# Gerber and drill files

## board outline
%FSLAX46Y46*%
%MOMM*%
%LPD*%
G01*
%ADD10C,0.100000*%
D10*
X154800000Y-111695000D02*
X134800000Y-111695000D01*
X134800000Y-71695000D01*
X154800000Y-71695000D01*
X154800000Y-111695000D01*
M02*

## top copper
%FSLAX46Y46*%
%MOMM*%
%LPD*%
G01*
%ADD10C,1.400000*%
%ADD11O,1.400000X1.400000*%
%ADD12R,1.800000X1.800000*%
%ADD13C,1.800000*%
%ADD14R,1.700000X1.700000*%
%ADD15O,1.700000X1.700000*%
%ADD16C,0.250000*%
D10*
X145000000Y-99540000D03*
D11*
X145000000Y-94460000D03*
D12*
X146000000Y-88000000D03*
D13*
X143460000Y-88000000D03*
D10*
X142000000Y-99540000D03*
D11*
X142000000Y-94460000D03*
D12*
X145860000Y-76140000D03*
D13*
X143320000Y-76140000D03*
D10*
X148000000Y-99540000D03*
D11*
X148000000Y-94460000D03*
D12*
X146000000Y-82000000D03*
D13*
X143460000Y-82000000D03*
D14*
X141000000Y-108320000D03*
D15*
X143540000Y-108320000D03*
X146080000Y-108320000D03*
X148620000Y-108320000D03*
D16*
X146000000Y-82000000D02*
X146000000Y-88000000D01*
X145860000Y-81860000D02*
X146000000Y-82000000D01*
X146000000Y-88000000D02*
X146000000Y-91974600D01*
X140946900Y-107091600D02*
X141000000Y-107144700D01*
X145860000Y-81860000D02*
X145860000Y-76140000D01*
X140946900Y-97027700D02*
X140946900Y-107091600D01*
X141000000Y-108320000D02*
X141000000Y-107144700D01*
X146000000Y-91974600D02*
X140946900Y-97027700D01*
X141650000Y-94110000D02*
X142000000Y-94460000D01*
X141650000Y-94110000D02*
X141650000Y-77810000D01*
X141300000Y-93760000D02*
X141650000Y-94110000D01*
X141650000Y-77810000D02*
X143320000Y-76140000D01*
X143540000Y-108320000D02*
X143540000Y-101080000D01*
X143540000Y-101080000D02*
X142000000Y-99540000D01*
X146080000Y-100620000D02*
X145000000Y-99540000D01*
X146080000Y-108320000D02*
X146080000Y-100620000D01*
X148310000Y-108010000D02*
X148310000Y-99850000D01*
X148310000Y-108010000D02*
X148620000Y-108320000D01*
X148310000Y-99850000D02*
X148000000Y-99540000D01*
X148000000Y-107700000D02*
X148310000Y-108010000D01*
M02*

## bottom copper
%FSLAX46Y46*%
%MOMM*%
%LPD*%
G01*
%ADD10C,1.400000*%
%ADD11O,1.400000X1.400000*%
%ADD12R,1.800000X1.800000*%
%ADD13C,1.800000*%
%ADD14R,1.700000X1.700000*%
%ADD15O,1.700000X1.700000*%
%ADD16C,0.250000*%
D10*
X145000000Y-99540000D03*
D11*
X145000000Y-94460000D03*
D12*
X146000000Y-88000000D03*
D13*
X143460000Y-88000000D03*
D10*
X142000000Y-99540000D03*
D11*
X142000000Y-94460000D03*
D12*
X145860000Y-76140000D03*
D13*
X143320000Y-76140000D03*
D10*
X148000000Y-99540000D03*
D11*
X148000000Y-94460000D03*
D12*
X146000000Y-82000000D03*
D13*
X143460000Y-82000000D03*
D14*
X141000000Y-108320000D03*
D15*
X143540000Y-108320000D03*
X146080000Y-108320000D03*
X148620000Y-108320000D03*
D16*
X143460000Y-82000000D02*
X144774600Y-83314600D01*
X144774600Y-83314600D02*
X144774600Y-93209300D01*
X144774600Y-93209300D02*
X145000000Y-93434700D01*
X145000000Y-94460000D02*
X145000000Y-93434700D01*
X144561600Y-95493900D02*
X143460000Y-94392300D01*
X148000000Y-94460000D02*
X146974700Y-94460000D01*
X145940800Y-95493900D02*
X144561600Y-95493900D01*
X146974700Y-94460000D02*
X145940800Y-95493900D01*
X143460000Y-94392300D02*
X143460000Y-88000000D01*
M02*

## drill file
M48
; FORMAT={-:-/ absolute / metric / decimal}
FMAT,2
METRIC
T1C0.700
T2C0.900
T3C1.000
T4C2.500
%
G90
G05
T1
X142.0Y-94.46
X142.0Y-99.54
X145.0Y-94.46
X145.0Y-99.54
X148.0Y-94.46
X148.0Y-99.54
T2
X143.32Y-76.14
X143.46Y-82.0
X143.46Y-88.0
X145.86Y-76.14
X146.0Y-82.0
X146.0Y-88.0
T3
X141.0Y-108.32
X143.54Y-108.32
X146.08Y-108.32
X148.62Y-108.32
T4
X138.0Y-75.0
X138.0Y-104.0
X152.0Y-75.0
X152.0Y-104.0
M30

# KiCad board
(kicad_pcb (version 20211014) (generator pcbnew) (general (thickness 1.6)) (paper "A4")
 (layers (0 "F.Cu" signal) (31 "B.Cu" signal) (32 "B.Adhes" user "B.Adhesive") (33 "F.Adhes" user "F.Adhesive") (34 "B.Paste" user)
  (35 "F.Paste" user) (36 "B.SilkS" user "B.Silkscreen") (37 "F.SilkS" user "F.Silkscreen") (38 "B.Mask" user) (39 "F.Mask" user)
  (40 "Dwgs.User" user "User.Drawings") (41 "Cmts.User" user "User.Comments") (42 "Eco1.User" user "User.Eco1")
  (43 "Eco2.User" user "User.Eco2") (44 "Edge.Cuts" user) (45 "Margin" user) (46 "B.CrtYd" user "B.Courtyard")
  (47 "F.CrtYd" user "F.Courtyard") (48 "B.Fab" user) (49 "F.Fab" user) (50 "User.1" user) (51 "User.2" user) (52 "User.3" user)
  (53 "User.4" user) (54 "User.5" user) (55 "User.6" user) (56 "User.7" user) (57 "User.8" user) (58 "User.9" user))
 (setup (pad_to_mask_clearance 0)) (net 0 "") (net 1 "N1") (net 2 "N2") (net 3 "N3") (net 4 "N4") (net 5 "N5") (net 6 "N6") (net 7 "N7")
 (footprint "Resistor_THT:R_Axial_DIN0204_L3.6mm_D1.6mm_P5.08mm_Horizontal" (layer "F.Cu") (at 145 99.54 90)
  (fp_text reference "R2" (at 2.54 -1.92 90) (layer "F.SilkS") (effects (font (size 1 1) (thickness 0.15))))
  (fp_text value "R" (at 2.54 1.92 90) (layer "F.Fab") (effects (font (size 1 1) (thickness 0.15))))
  (pad "1" thru_hole circle (at 0 0 90) (size 1.4 1.4) (drill 0.7) (layers *.Cu *.Mask) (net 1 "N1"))
  (pad "2" thru_hole oval (at 5.08 0 90) (size 1.4 1.4) (drill 0.7) (layers *.Cu *.Mask) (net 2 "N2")))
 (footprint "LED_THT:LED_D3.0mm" (layer "F.Cu") (at 146 88 180)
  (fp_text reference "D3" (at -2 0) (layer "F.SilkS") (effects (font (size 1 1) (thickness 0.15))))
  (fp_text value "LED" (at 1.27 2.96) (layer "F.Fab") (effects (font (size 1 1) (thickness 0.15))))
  (pad "1" thru_hole rect (at 0 0 180) (size 1.8 1.8) (drill 0.9) (layers *.Cu *.Mask) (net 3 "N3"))
  (pad "2" thru_hole circle (at 2.54 0 180) (size 1.8 1.8) (drill 0.9) (layers *.Cu *.Mask) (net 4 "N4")))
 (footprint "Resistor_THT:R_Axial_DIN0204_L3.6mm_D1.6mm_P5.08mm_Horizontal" (layer "F.Cu") (at 142 99.54 90)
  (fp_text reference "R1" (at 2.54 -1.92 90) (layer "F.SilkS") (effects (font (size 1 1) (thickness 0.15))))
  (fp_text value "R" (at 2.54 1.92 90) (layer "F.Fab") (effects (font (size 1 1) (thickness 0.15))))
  (pad "1" thru_hole circle (at 0 0 90) (size 1.4 1.4) (drill 0.7) (layers *.Cu *.Mask) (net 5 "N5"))
  (pad "2" thru_hole oval (at 5.08 0 90) (size 1.4 1.4) (drill 0.7) (layers *.Cu *.Mask) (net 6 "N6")))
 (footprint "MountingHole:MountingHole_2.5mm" (layer "F.Cu") (at 152 75)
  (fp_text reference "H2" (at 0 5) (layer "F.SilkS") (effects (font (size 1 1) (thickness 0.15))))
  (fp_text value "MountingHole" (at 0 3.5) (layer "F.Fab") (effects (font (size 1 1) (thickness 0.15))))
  (pad "" np_thru_hole circle (at 0 0) (size 2.5 2.5) (drill 2.5) (layers *.Cu *.Mask)))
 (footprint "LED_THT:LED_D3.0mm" (layer "F.Cu") (at 145.86 76.14 180)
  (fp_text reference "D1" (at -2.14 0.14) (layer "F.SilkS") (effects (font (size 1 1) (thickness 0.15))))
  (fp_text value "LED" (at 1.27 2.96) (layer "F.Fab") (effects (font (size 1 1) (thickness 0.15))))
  (pad "1" thru_hole rect (at 0 0 180) (size 1.8 1.8) (drill 0.9) (layers *.Cu *.Mask) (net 3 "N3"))
  (pad "2" thru_hole circle (at 2.54 0 180) (size 1.8 1.8) (drill 0.9) (layers *.Cu *.Mask) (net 6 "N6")))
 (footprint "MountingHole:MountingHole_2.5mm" (layer "F.Cu") (at 138 104)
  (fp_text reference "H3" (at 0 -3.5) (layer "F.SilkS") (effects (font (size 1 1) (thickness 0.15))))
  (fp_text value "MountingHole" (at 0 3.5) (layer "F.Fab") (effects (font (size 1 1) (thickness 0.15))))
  (pad "" np_thru_hole circle (at 0 0) (size 2.5 2.5) (drill 2.5) (layers *.Cu *.Mask)))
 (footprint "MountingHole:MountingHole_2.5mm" (layer "F.Cu") (at 152 104)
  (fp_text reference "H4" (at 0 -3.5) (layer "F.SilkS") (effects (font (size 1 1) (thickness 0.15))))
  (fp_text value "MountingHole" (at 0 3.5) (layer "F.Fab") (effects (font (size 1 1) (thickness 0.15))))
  (pad "" np_thru_hole circle (at 0 0) (size 2.5 2.5) (drill 2.5) (layers *.Cu *.Mask)))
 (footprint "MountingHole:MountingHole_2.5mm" (layer "F.Cu") (at 138 75)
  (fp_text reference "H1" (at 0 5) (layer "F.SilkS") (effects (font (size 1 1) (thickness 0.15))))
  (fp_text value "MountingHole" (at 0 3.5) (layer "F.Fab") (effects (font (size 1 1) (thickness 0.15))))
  (pad "" np_thru_hole circle (at 0 0) (size 2.5 2.5) (drill 2.5) (layers *.Cu *.Mask)))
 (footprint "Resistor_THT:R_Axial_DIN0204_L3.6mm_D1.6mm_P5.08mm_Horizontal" (layer "F.Cu") (at 148 99.54 90)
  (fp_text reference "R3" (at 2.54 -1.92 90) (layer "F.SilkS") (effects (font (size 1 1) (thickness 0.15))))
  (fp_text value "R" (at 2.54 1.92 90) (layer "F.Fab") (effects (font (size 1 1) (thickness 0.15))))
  (pad "1" thru_hole circle (at 0 0 90) (size 1.4 1.4) (drill 0.7) (layers *.Cu *.Mask) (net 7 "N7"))
  (pad "2" thru_hole oval (at 5.08 0 90) (size 1.4 1.4) (drill 0.7) (layers *.Cu *.Mask) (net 4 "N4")))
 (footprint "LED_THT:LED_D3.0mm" (layer "F.Cu") (at 146 82 180)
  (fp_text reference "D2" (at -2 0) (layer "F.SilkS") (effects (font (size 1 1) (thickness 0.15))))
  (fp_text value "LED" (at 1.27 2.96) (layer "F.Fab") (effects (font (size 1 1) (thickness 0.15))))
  (pad "1" thru_hole rect (at 0 0 180) (size 1.8 1.8) (drill 0.9) (layers *.Cu *.Mask) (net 3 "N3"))
  (pad "2" thru_hole circle (at 2.54 0 180) (size 1.8 1.8) (drill 0.9) (layers *.Cu *.Mask) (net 2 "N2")))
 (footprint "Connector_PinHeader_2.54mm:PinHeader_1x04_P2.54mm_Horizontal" (layer "B.Cu") (at 141 108.32 -90)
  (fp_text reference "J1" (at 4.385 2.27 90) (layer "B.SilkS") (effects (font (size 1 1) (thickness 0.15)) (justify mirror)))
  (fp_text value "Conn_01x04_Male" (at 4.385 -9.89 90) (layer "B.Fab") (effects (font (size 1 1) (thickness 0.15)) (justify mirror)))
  (pad "1" thru_hole rect (at 0 0 270) (size 1.7 1.7) (drill 1) (layers *.Cu *.Mask) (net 3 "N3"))
  (pad "2" thru_hole oval (at 0 -2.54 270) (size 1.7 1.7) (drill 1) (layers *.Cu *.Mask) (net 5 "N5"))
  (pad "3" thru_hole oval (at 0 -5.08 270) (size 1.7 1.7) (drill 1) (layers *.Cu *.Mask) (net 1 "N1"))
  (pad "4" thru_hole oval (at 0 -7.62 270) (size 1.7 1.7) (drill 1) (layers *.Cu *.Mask) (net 7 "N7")))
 (gr_poly (pts (xy 154.8 111.695) (xy 134.8 111.695) (xy 134.8 71.695) (xy 154.8 71.695)) (layer "Edge.Cuts") (width 0.1) (fill none))
 (segment (start 146 82) (end 146 88) (width 0.25) (layer "F.Cu") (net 3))
 (segment (start 145.86 81.86) (end 146 82) (width 0.25) (layer "F.Cu") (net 3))
 (segment (start 146 88) (end 146 91.9746) (width 0.25) (layer "F.Cu") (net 3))
 (segment (start 140.9469 107.0916) (end 141 107.1447) (width 0.25) (layer "F.Cu") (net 3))
 (segment (start 145.86 81.86) (end 145.86 76.14) (width 0.25) (layer "F.Cu") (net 3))
 (segment (start 140.9469 97.0277) (end 140.9469 107.0916) (width 0.25) (layer "F.Cu") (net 3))
 (segment (start 141 108.32) (end 141 107.1447) (width 0.25) (layer "F.Cu") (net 3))
 (segment (start 146 91.9746) (end 140.9469 97.0277) (width 0.25) (layer "F.Cu") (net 3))
 (segment (start 141.65 94.11) (end 142 94.46) (width 0.25) (layer "F.Cu") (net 6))
 (segment (start 141.65 94.11) (end 141.65 77.81) (width 0.25) (layer "F.Cu") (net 6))
 (segment (start 141.3 93.76) (end 141.65 94.11) (width 0.25) (layer "F.Cu") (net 6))
 (segment (start 141.65 77.81) (end 143.32 76.14) (width 0.25) (layer "F.Cu") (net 6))
 (segment (start 143.46 82) (end 144.7746 83.3146) (width 0.25) (layer "B.Cu") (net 2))
 (segment (start 144.7746 83.3146) (end 144.7746 93.2093) (width 0.25) (layer "B.Cu") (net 2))
 (segment (start 144.7746 93.2093) (end 145 93.4347) (width 0.25) (layer "B.Cu") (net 2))
 (segment (start 145 94.46) (end 145 93.4347) (width 0.25) (layer "B.Cu") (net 2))
 (segment (start 144.5616 95.4939) (end 143.46 94.3923) (width 0.25) (layer "B.Cu") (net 4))
 (segment (start 148 94.46) (end 146.9747 94.46) (width 0.25) (layer "B.Cu") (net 4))
 (segment (start 145.9408 95.4939) (end 144.5616 95.4939) (width 0.25) (layer "B.Cu") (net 4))
 (segment (start 146.9747 94.46) (end 145.9408 95.4939) (width 0.25) (layer "B.Cu") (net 4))
 (segment (start 143.46 94.3923) (end 143.46 88) (width 0.25) (layer "B.Cu") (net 4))
 (segment (start 143.54 108.32) (end 143.54 101.08) (width 0.25) (layer "F.Cu") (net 5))
 (segment (start 143.54 101.08) (end 142 99.54) (width 0.25) (layer "F.Cu") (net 5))
 (segment (start 146.08 100.62) (end 145 99.54) (width 0.25) (layer "F.Cu") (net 1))
 (segment (start 146.08 108.32) (end 146.08 100.62) (width 0.25) (layer "F.Cu") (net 1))
 (segment (start 148.31 108.01) (end 148.31 99.85) (width 0.25) (layer "F.Cu") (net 7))
 (segment (start 148.31 108.01) (end 148.62 108.32) (width 0.25) (layer "F.Cu") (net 7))
 (segment (start 148.31 99.85) (end 148 99.54) (width 0.25) (layer "F.Cu") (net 7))
 (segment (start 148 107.7) (end 148.31 108.01) (width 0.25) (layer "F.Cu") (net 7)))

